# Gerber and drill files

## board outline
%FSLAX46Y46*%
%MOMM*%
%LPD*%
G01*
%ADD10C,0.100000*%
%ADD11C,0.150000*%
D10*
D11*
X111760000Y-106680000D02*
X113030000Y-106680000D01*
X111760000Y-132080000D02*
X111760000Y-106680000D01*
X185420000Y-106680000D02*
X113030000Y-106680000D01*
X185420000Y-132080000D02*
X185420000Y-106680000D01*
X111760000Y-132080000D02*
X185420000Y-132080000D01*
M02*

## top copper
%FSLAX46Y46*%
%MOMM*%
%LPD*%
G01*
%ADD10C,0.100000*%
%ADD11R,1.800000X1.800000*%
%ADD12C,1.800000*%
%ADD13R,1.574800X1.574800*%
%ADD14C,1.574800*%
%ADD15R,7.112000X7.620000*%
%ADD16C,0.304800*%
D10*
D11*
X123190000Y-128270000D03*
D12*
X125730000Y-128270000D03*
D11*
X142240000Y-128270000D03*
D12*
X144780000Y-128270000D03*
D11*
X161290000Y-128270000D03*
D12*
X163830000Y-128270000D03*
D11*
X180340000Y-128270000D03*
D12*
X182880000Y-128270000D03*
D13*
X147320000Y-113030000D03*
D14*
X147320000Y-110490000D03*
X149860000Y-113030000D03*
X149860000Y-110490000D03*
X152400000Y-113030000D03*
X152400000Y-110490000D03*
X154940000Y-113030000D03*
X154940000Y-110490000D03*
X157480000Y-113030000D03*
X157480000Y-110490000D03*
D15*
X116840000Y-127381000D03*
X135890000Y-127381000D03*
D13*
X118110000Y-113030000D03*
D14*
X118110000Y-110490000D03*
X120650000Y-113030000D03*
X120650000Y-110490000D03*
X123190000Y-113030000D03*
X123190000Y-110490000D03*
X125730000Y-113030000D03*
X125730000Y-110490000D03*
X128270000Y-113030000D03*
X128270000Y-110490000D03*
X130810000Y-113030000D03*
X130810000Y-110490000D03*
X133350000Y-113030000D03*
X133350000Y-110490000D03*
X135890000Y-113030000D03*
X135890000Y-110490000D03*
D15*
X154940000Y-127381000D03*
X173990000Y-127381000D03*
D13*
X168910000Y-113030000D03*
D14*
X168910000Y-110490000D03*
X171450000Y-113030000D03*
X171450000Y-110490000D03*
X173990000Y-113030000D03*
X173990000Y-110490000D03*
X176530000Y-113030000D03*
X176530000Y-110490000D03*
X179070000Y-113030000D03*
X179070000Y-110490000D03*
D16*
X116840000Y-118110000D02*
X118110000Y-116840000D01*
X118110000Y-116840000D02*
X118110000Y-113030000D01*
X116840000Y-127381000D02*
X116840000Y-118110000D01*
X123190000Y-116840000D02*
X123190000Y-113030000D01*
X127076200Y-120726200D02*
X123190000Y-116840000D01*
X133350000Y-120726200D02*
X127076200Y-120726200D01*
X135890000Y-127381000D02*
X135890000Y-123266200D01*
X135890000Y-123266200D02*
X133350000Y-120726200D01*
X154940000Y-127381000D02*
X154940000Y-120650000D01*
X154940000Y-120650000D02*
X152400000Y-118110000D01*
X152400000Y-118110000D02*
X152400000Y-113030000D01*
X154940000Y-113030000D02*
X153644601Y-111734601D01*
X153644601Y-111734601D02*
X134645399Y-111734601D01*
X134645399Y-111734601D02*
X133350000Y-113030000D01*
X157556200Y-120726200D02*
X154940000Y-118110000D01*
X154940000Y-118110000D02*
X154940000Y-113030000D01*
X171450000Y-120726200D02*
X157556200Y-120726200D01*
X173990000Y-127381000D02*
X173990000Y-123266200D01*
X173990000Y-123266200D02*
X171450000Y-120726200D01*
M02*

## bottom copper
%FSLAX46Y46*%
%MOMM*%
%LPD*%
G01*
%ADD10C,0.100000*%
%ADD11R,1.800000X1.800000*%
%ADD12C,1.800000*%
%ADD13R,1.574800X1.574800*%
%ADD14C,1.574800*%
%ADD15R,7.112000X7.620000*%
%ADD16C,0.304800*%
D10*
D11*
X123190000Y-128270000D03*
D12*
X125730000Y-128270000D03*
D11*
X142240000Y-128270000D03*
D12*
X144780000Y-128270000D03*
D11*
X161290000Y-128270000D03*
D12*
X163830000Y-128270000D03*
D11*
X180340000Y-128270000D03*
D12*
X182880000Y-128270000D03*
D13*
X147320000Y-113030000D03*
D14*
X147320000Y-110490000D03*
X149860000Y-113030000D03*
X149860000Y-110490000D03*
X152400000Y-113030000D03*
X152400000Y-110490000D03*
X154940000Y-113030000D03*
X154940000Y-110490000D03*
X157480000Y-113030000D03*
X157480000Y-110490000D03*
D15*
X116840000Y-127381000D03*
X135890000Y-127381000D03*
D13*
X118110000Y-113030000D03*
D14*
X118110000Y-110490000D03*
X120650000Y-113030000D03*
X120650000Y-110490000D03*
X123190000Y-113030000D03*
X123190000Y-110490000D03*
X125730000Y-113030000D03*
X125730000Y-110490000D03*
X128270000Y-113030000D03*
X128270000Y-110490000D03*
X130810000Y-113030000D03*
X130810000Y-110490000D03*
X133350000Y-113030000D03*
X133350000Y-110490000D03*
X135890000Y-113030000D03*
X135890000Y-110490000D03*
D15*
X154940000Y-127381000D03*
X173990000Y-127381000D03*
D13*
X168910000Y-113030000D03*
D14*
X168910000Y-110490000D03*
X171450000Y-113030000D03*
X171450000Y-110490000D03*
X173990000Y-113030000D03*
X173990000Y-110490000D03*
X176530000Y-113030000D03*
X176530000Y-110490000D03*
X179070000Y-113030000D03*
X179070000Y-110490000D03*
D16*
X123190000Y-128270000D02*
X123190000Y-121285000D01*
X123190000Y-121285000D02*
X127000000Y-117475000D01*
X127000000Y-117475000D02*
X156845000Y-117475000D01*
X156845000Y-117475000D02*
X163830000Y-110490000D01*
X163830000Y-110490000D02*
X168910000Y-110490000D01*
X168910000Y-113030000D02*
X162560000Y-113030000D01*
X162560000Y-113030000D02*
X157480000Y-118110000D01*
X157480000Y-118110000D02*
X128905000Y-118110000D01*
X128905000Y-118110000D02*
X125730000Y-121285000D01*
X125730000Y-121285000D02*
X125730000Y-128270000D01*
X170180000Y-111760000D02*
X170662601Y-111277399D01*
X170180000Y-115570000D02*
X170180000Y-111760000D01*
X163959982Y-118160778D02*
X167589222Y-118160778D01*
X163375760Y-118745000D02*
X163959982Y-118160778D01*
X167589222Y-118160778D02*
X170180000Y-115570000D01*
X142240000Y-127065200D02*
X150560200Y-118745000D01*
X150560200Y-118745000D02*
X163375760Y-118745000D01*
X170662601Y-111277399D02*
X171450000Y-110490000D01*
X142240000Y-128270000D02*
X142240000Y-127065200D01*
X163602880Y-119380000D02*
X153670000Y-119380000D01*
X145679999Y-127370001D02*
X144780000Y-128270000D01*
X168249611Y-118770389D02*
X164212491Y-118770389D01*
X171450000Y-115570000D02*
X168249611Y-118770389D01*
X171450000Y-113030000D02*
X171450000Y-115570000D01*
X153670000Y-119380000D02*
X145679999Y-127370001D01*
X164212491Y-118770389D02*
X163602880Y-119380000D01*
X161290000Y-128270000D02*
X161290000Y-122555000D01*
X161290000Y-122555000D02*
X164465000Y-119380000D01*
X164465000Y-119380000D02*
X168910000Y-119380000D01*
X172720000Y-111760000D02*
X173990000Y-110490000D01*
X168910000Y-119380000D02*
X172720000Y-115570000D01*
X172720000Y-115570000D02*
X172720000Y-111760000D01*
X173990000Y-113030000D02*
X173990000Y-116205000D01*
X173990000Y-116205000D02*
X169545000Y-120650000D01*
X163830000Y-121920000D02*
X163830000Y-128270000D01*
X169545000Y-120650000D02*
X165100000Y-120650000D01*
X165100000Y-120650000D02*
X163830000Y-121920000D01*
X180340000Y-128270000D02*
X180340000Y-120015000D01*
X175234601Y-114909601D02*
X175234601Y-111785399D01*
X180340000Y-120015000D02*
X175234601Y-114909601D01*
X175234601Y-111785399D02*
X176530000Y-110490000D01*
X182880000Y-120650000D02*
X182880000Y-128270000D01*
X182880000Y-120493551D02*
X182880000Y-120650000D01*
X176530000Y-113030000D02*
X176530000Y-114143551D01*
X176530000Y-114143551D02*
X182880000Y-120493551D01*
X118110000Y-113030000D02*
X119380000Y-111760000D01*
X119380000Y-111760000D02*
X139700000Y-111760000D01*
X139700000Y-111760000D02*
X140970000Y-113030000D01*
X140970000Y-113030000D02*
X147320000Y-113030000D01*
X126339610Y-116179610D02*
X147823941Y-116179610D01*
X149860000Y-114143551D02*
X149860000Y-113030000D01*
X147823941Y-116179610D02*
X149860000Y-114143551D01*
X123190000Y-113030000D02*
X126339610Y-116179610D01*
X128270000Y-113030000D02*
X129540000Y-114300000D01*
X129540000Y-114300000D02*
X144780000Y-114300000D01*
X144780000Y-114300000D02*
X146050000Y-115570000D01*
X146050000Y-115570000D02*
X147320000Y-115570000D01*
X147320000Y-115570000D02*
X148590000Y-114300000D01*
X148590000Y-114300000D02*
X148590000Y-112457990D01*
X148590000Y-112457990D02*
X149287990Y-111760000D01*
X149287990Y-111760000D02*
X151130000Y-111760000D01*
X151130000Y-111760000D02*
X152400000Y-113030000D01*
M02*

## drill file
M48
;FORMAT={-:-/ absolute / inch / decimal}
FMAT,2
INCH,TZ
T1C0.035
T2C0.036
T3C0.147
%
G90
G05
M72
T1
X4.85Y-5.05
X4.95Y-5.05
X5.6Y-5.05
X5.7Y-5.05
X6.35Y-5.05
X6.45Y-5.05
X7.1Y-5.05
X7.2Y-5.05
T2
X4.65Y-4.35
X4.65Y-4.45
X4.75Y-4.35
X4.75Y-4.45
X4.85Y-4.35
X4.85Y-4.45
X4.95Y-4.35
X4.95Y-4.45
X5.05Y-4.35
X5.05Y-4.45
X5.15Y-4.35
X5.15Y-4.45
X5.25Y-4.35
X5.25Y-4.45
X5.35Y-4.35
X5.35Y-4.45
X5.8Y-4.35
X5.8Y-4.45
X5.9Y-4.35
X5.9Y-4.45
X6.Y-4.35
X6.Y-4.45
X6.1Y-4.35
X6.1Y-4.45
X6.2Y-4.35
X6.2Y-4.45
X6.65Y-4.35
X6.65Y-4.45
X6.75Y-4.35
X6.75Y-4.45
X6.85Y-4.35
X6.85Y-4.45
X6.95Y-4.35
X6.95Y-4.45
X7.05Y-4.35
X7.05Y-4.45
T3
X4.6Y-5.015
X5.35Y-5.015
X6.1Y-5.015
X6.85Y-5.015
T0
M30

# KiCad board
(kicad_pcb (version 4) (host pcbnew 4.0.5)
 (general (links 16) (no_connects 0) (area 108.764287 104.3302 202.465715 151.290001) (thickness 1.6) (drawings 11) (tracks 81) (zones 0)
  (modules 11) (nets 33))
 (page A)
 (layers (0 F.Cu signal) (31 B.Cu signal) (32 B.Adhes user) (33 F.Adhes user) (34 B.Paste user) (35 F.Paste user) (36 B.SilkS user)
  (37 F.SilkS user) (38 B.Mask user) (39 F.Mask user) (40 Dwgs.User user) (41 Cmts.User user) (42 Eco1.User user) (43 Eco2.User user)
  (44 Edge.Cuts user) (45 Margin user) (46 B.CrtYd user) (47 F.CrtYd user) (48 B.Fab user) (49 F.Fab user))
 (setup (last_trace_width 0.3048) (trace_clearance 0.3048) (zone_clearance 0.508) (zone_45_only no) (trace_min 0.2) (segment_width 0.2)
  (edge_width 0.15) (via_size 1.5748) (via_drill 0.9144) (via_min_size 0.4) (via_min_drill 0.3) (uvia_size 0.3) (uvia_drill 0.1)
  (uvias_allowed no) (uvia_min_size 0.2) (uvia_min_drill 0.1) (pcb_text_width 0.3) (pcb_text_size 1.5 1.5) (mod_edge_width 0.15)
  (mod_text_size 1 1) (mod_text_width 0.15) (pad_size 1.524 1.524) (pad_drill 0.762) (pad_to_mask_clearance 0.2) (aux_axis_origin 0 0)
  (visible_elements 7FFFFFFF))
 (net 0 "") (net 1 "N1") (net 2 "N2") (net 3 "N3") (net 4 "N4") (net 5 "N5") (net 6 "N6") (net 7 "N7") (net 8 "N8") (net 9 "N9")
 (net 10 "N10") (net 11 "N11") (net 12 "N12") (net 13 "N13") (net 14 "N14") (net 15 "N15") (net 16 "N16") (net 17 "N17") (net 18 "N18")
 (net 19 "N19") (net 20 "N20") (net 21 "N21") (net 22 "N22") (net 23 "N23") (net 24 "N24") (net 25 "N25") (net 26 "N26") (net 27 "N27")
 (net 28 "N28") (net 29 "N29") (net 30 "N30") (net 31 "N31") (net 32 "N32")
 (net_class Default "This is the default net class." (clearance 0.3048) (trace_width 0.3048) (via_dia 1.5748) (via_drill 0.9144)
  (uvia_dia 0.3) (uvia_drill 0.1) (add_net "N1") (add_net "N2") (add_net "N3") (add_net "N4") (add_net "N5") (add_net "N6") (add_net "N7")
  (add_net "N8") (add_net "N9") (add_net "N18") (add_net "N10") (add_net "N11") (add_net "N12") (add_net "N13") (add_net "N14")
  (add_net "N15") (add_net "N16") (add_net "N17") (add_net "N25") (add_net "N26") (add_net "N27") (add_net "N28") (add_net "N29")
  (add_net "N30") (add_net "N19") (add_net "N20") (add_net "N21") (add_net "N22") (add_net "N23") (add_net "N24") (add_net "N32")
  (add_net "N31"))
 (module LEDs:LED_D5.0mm (layer F.Cu) (at 123.19 128.27)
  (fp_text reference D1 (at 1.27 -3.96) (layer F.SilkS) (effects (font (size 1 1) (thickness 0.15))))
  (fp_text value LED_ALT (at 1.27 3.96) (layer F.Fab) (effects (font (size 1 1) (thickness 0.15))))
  (pad 1 thru_hole rect (at 0 0) (size 1.8 1.8) (drill 0.9) (layers *.Cu *.Mask) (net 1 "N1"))
  (pad 2 thru_hole circle (at 2.54 0) (size 1.8 1.8) (drill 0.9) (layers *.Cu *.Mask) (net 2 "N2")))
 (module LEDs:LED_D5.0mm (layer F.Cu) (at 142.24 128.27)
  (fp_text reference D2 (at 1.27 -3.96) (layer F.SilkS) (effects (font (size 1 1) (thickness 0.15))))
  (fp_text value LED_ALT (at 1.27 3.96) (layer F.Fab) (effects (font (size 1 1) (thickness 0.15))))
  (pad 1 thru_hole rect (at 0 0) (size 1.8 1.8) (drill 0.9) (layers *.Cu *.Mask) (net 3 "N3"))
  (pad 2 thru_hole circle (at 2.54 0) (size 1.8 1.8) (drill 0.9) (layers *.Cu *.Mask) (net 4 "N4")))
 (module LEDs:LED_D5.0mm (layer F.Cu) (at 161.29 128.27)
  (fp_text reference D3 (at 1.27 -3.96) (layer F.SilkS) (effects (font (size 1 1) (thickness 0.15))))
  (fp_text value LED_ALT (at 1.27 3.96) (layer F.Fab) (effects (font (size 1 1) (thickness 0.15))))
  (pad 1 thru_hole rect (at 0 0) (size 1.8 1.8) (drill 0.9) (layers *.Cu *.Mask) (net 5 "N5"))
  (pad 2 thru_hole circle (at 2.54 0) (size 1.8 1.8) (drill 0.9) (layers *.Cu *.Mask) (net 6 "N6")))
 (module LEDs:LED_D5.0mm (layer F.Cu) (at 180.34 128.27)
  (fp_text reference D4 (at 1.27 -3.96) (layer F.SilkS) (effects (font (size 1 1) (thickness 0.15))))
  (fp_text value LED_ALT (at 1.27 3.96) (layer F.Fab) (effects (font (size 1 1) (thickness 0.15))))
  (pad 1 thru_hole rect (at 0 0) (size 1.8 1.8) (drill 0.9) (layers *.Cu *.Mask) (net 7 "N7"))
  (pad 2 thru_hole circle (at 2.54 0) (size 1.8 1.8) (drill 0.9) (layers *.Cu *.Mask) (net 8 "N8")))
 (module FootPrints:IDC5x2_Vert (layer F.Cu) (at 152.4 111.76 180)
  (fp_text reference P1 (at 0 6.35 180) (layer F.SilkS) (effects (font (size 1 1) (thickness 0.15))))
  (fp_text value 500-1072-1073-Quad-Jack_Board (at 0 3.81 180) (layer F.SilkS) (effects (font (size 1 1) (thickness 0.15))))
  (pad 1 thru_hole rect (at 5.08 -1.27 180) (size 1.5748 1.5748) (drill 0.9144) (layers *.Cu *.Mask F.SilkS) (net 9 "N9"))
  (pad 2 thru_hole circle (at 5.08 1.27 180) (size 1.5748 1.5748) (drill 0.9144) (layers *.Cu *.Mask F.SilkS) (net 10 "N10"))
  (pad 3 thru_hole circle (at 2.54 -1.27 180) (size 1.5748 1.5748) (drill 0.9144) (layers *.Cu *.Mask F.SilkS) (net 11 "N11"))
  (pad 4 thru_hole circle (at 2.54 1.27 180) (size 1.5748 1.5748) (drill 0.9144) (layers *.Cu *.Mask F.SilkS) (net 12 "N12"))
  (pad 5 thru_hole circle (at 0 -1.27 180) (size 1.5748 1.5748) (drill 0.9144) (layers *.Cu *.Mask F.SilkS) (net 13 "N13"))
  (pad 6 thru_hole circle (at 0 1.27 180) (size 1.5748 1.5748) (drill 0.9144) (layers *.Cu *.Mask F.SilkS) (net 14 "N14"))
  (pad 7 thru_hole circle (at -2.54 -1.27 180) (size 1.5748 1.5748) (drill 0.9144) (layers *.Cu *.Mask F.SilkS) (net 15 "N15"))
  (pad 8 thru_hole circle (at -2.54 1.27 180) (size 1.5748 1.5748) (drill 0.9144) (layers *.Cu *.Mask F.SilkS) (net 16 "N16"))
  (pad 9 thru_hole circle (at -5.08 -1.27 180) (size 1.5748 1.5748) (drill 0.9144) (layers *.Cu *.Mask F.SilkS) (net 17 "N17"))
  (pad 10 thru_hole circle (at -5.08 1.27 180) (size 1.5748 1.5748) (drill 0.9144) (layers *.Cu *.Mask F.SilkS) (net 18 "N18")))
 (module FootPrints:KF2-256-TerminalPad (layer F.Cu) (at 116.84 132.08)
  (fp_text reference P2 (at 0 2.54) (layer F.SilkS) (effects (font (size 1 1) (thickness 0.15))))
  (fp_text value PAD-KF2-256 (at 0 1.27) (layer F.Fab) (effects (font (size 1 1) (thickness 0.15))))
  (pad 1 thru_hole rect (at 0 -4.699) (size 7.112 7.62) (drill 3.7338) (layers *.Cu *.Mask F.SilkS) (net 9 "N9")))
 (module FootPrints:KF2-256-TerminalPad (layer F.Cu) (at 135.89 132.08)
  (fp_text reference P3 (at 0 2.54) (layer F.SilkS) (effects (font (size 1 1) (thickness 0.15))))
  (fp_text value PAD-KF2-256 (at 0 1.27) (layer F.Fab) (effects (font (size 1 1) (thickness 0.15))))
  (pad 1 thru_hole rect (at 0 -4.699) (size 7.112 7.62) (drill 3.7338) (layers *.Cu *.Mask F.SilkS) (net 11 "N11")))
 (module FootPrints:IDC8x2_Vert (layer F.Cu) (at 127 111.76 180)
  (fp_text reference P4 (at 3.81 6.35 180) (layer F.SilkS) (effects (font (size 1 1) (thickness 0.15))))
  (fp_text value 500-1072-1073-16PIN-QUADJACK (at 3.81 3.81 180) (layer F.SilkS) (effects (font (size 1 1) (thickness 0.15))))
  (pad 1 thru_hole rect (at 8.89 -1.27 180) (size 1.5748 1.5748) (drill 0.9144) (layers *.Cu *.Mask F.SilkS) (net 9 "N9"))
  (pad 2 thru_hole circle (at 8.89 1.27 180) (size 1.5748 1.5748) (drill 0.9144) (layers *.Cu *.Mask F.SilkS) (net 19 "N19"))
  (pad 3 thru_hole circle (at 6.35 -1.27 180) (size 1.5748 1.5748) (drill 0.9144) (layers *.Cu *.Mask F.SilkS) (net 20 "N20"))
  (pad 4 thru_hole circle (at 6.35 1.27 180) (size 1.5748 1.5748) (drill 0.9144) (layers *.Cu *.Mask F.SilkS) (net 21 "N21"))
  (pad 5 thru_hole circle (at 3.81 -1.27 180) (size 1.5748 1.5748) (drill 0.9144) (layers *.Cu *.Mask F.SilkS) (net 11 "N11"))
  (pad 6 thru_hole circle (at 3.81 1.27 180) (size 1.5748 1.5748) (drill 0.9144) (layers *.Cu *.Mask F.SilkS) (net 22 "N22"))
  (pad 7 thru_hole circle (at 1.27 -1.27 180) (size 1.5748 1.5748) (drill 0.9144) (layers *.Cu *.Mask F.SilkS) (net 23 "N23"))
  (pad 8 thru_hole circle (at 1.27 1.27 180) (size 1.5748 1.5748) (drill 0.9144) (layers *.Cu *.Mask F.SilkS) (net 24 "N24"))
  (pad 9 thru_hole circle (at -1.27 -1.27 180) (size 1.5748 1.5748) (drill 0.9144) (layers *.Cu *.Mask F.SilkS) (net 13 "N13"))
  (pad 10 thru_hole circle (at -1.27 1.27 180) (size 1.5748 1.5748) (drill 0.9144) (layers *.Cu *.Mask F.SilkS) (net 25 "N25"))
  (pad 11 thru_hole circle (at -3.81 -1.27 180) (size 1.5748 1.5748) (drill 0.9144) (layers *.Cu *.Mask F.SilkS) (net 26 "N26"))
  (pad 12 thru_hole circle (at -3.81 1.27 180) (size 1.5748 1.5748) (drill 0.9144) (layers *.Cu *.Mask F.SilkS) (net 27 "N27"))
  (pad 13 thru_hole circle (at -6.35 -1.27 180) (size 1.5748 1.5748) (drill 0.9144) (layers *.Cu *.Mask F.SilkS) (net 15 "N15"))
  (pad 14 thru_hole circle (at -6.35 1.27 180) (size 1.5748 1.5748) (drill 0.9144) (layers *.Cu *.Mask F.SilkS) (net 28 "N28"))
  (pad 15 thru_hole circle (at -8.89 -1.27 180) (size 1.5748 1.5748) (drill 0.9144) (layers *.Cu *.Mask F.SilkS) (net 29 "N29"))
  (pad 16 thru_hole circle (at -8.89 1.27 180) (size 1.5748 1.5748) (drill 0.9144) (layers *.Cu *.Mask F.SilkS) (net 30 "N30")))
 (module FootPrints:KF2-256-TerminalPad (layer F.Cu) (at 154.94 132.08)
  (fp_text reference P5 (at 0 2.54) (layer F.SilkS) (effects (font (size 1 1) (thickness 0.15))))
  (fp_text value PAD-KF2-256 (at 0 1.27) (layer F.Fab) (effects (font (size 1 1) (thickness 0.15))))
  (pad 1 thru_hole rect (at 0 -4.699) (size 7.112 7.62) (drill 3.7338) (layers *.Cu *.Mask F.SilkS) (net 13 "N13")))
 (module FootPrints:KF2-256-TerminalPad (layer F.Cu) (at 173.99 132.08)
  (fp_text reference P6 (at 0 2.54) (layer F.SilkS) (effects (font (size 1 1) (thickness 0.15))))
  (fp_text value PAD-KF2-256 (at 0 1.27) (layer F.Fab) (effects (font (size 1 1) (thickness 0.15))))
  (pad 1 thru_hole rect (at 0 -4.699) (size 7.112 7.62) (drill 3.7338) (layers *.Cu *.Mask F.SilkS) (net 15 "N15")))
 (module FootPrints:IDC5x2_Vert (layer F.Cu) (at 173.99 111.76 180)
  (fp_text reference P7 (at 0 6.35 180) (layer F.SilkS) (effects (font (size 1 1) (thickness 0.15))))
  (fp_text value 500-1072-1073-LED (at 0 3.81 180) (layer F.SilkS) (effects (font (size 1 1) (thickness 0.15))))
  (pad 1 thru_hole rect (at 5.08 -1.27 180) (size 1.5748 1.5748) (drill 0.9144) (layers *.Cu *.Mask F.SilkS) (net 2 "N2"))
  (pad 2 thru_hole circle (at 5.08 1.27 180) (size 1.5748 1.5748) (drill 0.9144) (layers *.Cu *.Mask F.SilkS) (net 1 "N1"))
  (pad 3 thru_hole circle (at 2.54 -1.27 180) (size 1.5748 1.5748) (drill 0.9144) (layers *.Cu *.Mask F.SilkS) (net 4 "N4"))
  (pad 4 thru_hole circle (at 2.54 1.27 180) (size 1.5748 1.5748) (drill 0.9144) (layers *.Cu *.Mask F.SilkS) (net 3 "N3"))
  (pad 5 thru_hole circle (at 0 -1.27 180) (size 1.5748 1.5748) (drill 0.9144) (layers *.Cu *.Mask F.SilkS) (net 6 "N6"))
  (pad 6 thru_hole circle (at 0 1.27 180) (size 1.5748 1.5748) (drill 0.9144) (layers *.Cu *.Mask F.SilkS) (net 5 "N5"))
  (pad 7 thru_hole circle (at -2.54 -1.27 180) (size 1.5748 1.5748) (drill 0.9144) (layers *.Cu *.Mask F.SilkS) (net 8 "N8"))
  (pad 8 thru_hole circle (at -2.54 1.27 180) (size 1.5748 1.5748) (drill 0.9144) (layers *.Cu *.Mask F.SilkS) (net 7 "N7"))
  (pad 9 thru_hole circle (at -5.08 -1.27 180) (size 1.5748 1.5748) (drill 0.9144) (layers *.Cu *.Mask F.SilkS) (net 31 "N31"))
  (pad 10 thru_hole circle (at -5.08 1.27 180) (size 1.5748 1.5748) (drill 0.9144) (layers *.Cu *.Mask F.SilkS) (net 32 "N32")))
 (gr_line (start 111.76 106.68) (end 113.03 106.68) (angle 90) (layer Edge.Cuts) (width 0.15))
 (gr_line (start 111.76 132.08) (end 111.76 106.68) (angle 90) (layer Edge.Cuts) (width 0.15))
 (gr_line (start 185.42 106.68) (end 113.03 106.68) (angle 90) (layer Edge.Cuts) (width 0.15))
 (gr_line (start 185.42 132.08) (end 185.42 106.68) (angle 90) (layer Edge.Cuts) (width 0.15))
 (gr_line (start 111.76 132.08) (end 185.42 132.08) (angle 90) (layer Edge.Cuts) (width 0.15))
 (segment (start 123.19 128.27) (end 123.19 121.285) (width 0.3048) (layer B.Cu) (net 1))
 (segment (start 123.19 121.285) (end 127 117.475) (width 0.3048) (layer B.Cu) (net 1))
 (segment (start 127 117.475) (end 156.845 117.475) (width 0.3048) (layer B.Cu) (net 1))
 (segment (start 156.845 117.475) (end 163.83 110.49) (width 0.3048) (layer B.Cu) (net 1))
 (segment (start 163.83 110.49) (end 168.91 110.49) (width 0.3048) (layer B.Cu) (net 1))
 (segment (start 168.91 113.03) (end 162.56 113.03) (width 0.3048) (layer B.Cu) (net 2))
 (segment (start 162.56 113.03) (end 157.48 118.11) (width 0.3048) (layer B.Cu) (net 2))
 (segment (start 157.48 118.11) (end 128.905 118.11) (width 0.3048) (layer B.Cu) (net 2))
 (segment (start 128.905 118.11) (end 125.73 121.285) (width 0.3048) (layer B.Cu) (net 2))
 (segment (start 125.73 121.285) (end 125.73 128.27) (width 0.3048) (layer B.Cu) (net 2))
 (segment (start 170.18 111.76) (end 170.662601 111.277399) (width 0.3048) (layer B.Cu) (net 3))
 (segment (start 170.18 115.57) (end 170.18 111.76) (width 0.3048) (layer B.Cu) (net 3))
 (segment (start 163.959982 118.160778) (end 167.589222 118.160778) (width 0.3048) (layer B.Cu) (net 3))
 (segment (start 163.37576 118.745) (end 163.959982 118.160778) (width 0.3048) (layer B.Cu) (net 3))
 (segment (start 167.589222 118.160778) (end 170.18 115.57) (width 0.3048) (layer B.Cu) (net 3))
 (segment (start 142.24 127.0652) (end 150.5602 118.745) (width 0.3048) (layer B.Cu) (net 3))
 (segment (start 150.5602 118.745) (end 163.37576 118.745) (width 0.3048) (layer B.Cu) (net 3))
 (segment (start 170.662601 111.277399) (end 171.45 110.49) (width 0.3048) (layer B.Cu) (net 3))
 (segment (start 142.24 128.27) (end 142.24 127.0652) (width 0.3048) (layer B.Cu) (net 3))
 (segment (start 163.60288 119.38) (end 153.67 119.38) (width 0.3048) (layer B.Cu) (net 4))
 (segment (start 145.679999 127.370001) (end 144.78 128.27) (width 0.3048) (layer B.Cu) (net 4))
 (segment (start 168.249611 118.770389) (end 164.212491 118.770389) (width 0.3048) (layer B.Cu) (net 4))
 (segment (start 171.45 115.57) (end 168.249611 118.770389) (width 0.3048) (layer B.Cu) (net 4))
 (segment (start 171.45 113.03) (end 171.45 115.57) (width 0.3048) (layer B.Cu) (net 4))
 (segment (start 153.67 119.38) (end 145.679999 127.370001) (width 0.3048) (layer B.Cu) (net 4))
 (segment (start 164.212491 118.770389) (end 163.60288 119.38) (width 0.3048) (layer B.Cu) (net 4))
 (segment (start 161.29 128.27) (end 161.29 122.555) (width 0.3048) (layer B.Cu) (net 5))
 (segment (start 161.29 122.555) (end 164.465 119.38) (width 0.3048) (layer B.Cu) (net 5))
 (segment (start 164.465 119.38) (end 168.91 119.38) (width 0.3048) (layer B.Cu) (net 5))
 (segment (start 172.72 111.76) (end 173.99 110.49) (width 0.3048) (layer B.Cu) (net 5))
 (segment (start 168.91 119.38) (end 172.72 115.57) (width 0.3048) (layer B.Cu) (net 5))
 (segment (start 172.72 115.57) (end 172.72 111.76) (width 0.3048) (layer B.Cu) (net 5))
 (segment (start 173.99 113.03) (end 173.99 116.205) (width 0.3048) (layer B.Cu) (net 6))
 (segment (start 173.99 116.205) (end 169.545 120.65) (width 0.3048) (layer B.Cu) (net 6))
 (segment (start 163.83 121.92) (end 163.83 128.27) (width 0.3048) (layer B.Cu) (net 6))
 (segment (start 169.545 120.65) (end 165.1 120.65) (width 0.3048) (layer B.Cu) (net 6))
 (segment (start 165.1 120.65) (end 163.83 121.92) (width 0.3048) (layer B.Cu) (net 6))
 (segment (start 180.34 128.27) (end 180.34 120.015) (width 0.3048) (layer B.Cu) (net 7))
 (segment (start 175.234601 114.909601) (end 175.234601 111.785399) (width 0.3048) (layer B.Cu) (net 7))
 (segment (start 180.34 120.015) (end 175.234601 114.909601) (width 0.3048) (layer B.Cu) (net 7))
 (segment (start 175.234601 111.785399) (end 176.53 110.49) (width 0.3048) (layer B.Cu) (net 7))
 (segment (start 182.88 120.65) (end 182.88 128.27) (width 0.3048) (layer B.Cu) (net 8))
 (segment (start 182.88 120.493551) (end 182.88 120.65) (width 0.3048) (layer B.Cu) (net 8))
 (segment (start 176.53 113.03) (end 176.53 114.143551) (width 0.3048) (layer B.Cu) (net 8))
 (segment (start 176.53 114.143551) (end 182.88 120.493551) (width 0.3048) (layer B.Cu) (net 8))
 (segment (start 118.11 113.03) (end 119.38 111.76) (width 0.3048) (layer B.Cu) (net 9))
 (segment (start 119.38 111.76) (end 139.7 111.76) (width 0.3048) (layer B.Cu) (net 9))
 (segment (start 139.7 111.76) (end 140.97 113.03) (width 0.3048) (layer B.Cu) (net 9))
 (segment (start 140.97 113.03) (end 147.32 113.03) (width 0.3048) (layer B.Cu) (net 9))
 (segment (start 116.84 118.11) (end 118.11 116.84) (width 0.3048) (layer F.Cu) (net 9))
 (segment (start 118.11 116.84) (end 118.11 113.03) (width 0.3048) (layer F.Cu) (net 9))
 (segment (start 116.84 127.381) (end 116.84 118.11) (width 0.3048) (layer F.Cu) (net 9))
 (segment (start 126.33961 116.17961) (end 147.823941 116.17961) (width 0.3048) (layer B.Cu) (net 11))
 (segment (start 149.86 114.143551) (end 149.86 113.03) (width 0.3048) (layer B.Cu) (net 11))
 (segment (start 147.823941 116.17961) (end 149.86 114.143551) (width 0.3048) (layer B.Cu) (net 11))
 (segment (start 123.19 113.03) (end 126.33961 116.17961) (width 0.3048) (layer B.Cu) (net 11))
 (segment (start 123.19 116.84) (end 123.19 113.03) (width 0.3048) (layer F.Cu) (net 11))
 (segment (start 127.0762 120.7262) (end 123.19 116.84) (width 0.3048) (layer F.Cu) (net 11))
 (segment (start 133.35 120.7262) (end 127.0762 120.7262) (width 0.3048) (layer F.Cu) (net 11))
 (segment (start 135.89 127.381) (end 135.89 123.2662) (width 0.3048) (layer F.Cu) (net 11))
 (segment (start 135.89 123.2662) (end 133.35 120.7262) (width 0.3048) (layer F.Cu) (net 11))
 (segment (start 128.27 113.03) (end 129.54 114.3) (width 0.3048) (layer B.Cu) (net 13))
 (segment (start 129.54 114.3) (end 144.78 114.3) (width 0.3048) (layer B.Cu) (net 13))
 (segment (start 144.78 114.3) (end 146.05 115.57) (width 0.3048) (layer B.Cu) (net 13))
 (segment (start 146.05 115.57) (end 147.32 115.57) (width 0.3048) (layer B.Cu) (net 13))
 (segment (start 147.32 115.57) (end 148.59 114.3) (width 0.3048) (layer B.Cu) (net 13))
 (segment (start 148.59 114.3) (end 148.59 112.45799) (width 0.3048) (layer B.Cu) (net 13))
 (segment (start 148.59 112.45799) (end 149.28799 111.76) (width 0.3048) (layer B.Cu) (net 13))
 (segment (start 149.28799 111.76) (end 151.13 111.76) (width 0.3048) (layer B.Cu) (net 13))
 (segment (start 151.13 111.76) (end 152.4 113.03) (width 0.3048) (layer B.Cu) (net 13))
 (segment (start 154.94 127.381) (end 154.94 120.65) (width 0.3048) (layer F.Cu) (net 13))
 (segment (start 154.94 120.65) (end 152.4 118.11) (width 0.3048) (layer F.Cu) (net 13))
 (segment (start 152.4 118.11) (end 152.4 113.03) (width 0.3048) (layer F.Cu) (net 13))
 (segment (start 154.94 113.03) (end 153.644601 111.734601) (width 0.3048) (layer F.Cu) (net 15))
 (segment (start 153.644601 111.734601) (end 134.645399 111.734601) (width 0.3048) (layer F.Cu) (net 15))
 (segment (start 134.645399 111.734601) (end 133.35 113.03) (width 0.3048) (layer F.Cu) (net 15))
 (segment (start 157.5562 120.7262) (end 154.94 118.11) (width 0.3048) (layer F.Cu) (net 15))
 (segment (start 154.94 118.11) (end 154.94 113.03) (width 0.3048) (layer F.Cu) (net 15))
 (segment (start 171.45 120.7262) (end 157.5562 120.7262) (width 0.3048) (layer F.Cu) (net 15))
 (segment (start 173.99 127.381) (end 173.99 123.2662) (width 0.3048) (layer F.Cu) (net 15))
 (segment (start 173.99 123.2662) (end 171.45 120.7262) (width 0.3048) (layer F.Cu) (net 15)))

